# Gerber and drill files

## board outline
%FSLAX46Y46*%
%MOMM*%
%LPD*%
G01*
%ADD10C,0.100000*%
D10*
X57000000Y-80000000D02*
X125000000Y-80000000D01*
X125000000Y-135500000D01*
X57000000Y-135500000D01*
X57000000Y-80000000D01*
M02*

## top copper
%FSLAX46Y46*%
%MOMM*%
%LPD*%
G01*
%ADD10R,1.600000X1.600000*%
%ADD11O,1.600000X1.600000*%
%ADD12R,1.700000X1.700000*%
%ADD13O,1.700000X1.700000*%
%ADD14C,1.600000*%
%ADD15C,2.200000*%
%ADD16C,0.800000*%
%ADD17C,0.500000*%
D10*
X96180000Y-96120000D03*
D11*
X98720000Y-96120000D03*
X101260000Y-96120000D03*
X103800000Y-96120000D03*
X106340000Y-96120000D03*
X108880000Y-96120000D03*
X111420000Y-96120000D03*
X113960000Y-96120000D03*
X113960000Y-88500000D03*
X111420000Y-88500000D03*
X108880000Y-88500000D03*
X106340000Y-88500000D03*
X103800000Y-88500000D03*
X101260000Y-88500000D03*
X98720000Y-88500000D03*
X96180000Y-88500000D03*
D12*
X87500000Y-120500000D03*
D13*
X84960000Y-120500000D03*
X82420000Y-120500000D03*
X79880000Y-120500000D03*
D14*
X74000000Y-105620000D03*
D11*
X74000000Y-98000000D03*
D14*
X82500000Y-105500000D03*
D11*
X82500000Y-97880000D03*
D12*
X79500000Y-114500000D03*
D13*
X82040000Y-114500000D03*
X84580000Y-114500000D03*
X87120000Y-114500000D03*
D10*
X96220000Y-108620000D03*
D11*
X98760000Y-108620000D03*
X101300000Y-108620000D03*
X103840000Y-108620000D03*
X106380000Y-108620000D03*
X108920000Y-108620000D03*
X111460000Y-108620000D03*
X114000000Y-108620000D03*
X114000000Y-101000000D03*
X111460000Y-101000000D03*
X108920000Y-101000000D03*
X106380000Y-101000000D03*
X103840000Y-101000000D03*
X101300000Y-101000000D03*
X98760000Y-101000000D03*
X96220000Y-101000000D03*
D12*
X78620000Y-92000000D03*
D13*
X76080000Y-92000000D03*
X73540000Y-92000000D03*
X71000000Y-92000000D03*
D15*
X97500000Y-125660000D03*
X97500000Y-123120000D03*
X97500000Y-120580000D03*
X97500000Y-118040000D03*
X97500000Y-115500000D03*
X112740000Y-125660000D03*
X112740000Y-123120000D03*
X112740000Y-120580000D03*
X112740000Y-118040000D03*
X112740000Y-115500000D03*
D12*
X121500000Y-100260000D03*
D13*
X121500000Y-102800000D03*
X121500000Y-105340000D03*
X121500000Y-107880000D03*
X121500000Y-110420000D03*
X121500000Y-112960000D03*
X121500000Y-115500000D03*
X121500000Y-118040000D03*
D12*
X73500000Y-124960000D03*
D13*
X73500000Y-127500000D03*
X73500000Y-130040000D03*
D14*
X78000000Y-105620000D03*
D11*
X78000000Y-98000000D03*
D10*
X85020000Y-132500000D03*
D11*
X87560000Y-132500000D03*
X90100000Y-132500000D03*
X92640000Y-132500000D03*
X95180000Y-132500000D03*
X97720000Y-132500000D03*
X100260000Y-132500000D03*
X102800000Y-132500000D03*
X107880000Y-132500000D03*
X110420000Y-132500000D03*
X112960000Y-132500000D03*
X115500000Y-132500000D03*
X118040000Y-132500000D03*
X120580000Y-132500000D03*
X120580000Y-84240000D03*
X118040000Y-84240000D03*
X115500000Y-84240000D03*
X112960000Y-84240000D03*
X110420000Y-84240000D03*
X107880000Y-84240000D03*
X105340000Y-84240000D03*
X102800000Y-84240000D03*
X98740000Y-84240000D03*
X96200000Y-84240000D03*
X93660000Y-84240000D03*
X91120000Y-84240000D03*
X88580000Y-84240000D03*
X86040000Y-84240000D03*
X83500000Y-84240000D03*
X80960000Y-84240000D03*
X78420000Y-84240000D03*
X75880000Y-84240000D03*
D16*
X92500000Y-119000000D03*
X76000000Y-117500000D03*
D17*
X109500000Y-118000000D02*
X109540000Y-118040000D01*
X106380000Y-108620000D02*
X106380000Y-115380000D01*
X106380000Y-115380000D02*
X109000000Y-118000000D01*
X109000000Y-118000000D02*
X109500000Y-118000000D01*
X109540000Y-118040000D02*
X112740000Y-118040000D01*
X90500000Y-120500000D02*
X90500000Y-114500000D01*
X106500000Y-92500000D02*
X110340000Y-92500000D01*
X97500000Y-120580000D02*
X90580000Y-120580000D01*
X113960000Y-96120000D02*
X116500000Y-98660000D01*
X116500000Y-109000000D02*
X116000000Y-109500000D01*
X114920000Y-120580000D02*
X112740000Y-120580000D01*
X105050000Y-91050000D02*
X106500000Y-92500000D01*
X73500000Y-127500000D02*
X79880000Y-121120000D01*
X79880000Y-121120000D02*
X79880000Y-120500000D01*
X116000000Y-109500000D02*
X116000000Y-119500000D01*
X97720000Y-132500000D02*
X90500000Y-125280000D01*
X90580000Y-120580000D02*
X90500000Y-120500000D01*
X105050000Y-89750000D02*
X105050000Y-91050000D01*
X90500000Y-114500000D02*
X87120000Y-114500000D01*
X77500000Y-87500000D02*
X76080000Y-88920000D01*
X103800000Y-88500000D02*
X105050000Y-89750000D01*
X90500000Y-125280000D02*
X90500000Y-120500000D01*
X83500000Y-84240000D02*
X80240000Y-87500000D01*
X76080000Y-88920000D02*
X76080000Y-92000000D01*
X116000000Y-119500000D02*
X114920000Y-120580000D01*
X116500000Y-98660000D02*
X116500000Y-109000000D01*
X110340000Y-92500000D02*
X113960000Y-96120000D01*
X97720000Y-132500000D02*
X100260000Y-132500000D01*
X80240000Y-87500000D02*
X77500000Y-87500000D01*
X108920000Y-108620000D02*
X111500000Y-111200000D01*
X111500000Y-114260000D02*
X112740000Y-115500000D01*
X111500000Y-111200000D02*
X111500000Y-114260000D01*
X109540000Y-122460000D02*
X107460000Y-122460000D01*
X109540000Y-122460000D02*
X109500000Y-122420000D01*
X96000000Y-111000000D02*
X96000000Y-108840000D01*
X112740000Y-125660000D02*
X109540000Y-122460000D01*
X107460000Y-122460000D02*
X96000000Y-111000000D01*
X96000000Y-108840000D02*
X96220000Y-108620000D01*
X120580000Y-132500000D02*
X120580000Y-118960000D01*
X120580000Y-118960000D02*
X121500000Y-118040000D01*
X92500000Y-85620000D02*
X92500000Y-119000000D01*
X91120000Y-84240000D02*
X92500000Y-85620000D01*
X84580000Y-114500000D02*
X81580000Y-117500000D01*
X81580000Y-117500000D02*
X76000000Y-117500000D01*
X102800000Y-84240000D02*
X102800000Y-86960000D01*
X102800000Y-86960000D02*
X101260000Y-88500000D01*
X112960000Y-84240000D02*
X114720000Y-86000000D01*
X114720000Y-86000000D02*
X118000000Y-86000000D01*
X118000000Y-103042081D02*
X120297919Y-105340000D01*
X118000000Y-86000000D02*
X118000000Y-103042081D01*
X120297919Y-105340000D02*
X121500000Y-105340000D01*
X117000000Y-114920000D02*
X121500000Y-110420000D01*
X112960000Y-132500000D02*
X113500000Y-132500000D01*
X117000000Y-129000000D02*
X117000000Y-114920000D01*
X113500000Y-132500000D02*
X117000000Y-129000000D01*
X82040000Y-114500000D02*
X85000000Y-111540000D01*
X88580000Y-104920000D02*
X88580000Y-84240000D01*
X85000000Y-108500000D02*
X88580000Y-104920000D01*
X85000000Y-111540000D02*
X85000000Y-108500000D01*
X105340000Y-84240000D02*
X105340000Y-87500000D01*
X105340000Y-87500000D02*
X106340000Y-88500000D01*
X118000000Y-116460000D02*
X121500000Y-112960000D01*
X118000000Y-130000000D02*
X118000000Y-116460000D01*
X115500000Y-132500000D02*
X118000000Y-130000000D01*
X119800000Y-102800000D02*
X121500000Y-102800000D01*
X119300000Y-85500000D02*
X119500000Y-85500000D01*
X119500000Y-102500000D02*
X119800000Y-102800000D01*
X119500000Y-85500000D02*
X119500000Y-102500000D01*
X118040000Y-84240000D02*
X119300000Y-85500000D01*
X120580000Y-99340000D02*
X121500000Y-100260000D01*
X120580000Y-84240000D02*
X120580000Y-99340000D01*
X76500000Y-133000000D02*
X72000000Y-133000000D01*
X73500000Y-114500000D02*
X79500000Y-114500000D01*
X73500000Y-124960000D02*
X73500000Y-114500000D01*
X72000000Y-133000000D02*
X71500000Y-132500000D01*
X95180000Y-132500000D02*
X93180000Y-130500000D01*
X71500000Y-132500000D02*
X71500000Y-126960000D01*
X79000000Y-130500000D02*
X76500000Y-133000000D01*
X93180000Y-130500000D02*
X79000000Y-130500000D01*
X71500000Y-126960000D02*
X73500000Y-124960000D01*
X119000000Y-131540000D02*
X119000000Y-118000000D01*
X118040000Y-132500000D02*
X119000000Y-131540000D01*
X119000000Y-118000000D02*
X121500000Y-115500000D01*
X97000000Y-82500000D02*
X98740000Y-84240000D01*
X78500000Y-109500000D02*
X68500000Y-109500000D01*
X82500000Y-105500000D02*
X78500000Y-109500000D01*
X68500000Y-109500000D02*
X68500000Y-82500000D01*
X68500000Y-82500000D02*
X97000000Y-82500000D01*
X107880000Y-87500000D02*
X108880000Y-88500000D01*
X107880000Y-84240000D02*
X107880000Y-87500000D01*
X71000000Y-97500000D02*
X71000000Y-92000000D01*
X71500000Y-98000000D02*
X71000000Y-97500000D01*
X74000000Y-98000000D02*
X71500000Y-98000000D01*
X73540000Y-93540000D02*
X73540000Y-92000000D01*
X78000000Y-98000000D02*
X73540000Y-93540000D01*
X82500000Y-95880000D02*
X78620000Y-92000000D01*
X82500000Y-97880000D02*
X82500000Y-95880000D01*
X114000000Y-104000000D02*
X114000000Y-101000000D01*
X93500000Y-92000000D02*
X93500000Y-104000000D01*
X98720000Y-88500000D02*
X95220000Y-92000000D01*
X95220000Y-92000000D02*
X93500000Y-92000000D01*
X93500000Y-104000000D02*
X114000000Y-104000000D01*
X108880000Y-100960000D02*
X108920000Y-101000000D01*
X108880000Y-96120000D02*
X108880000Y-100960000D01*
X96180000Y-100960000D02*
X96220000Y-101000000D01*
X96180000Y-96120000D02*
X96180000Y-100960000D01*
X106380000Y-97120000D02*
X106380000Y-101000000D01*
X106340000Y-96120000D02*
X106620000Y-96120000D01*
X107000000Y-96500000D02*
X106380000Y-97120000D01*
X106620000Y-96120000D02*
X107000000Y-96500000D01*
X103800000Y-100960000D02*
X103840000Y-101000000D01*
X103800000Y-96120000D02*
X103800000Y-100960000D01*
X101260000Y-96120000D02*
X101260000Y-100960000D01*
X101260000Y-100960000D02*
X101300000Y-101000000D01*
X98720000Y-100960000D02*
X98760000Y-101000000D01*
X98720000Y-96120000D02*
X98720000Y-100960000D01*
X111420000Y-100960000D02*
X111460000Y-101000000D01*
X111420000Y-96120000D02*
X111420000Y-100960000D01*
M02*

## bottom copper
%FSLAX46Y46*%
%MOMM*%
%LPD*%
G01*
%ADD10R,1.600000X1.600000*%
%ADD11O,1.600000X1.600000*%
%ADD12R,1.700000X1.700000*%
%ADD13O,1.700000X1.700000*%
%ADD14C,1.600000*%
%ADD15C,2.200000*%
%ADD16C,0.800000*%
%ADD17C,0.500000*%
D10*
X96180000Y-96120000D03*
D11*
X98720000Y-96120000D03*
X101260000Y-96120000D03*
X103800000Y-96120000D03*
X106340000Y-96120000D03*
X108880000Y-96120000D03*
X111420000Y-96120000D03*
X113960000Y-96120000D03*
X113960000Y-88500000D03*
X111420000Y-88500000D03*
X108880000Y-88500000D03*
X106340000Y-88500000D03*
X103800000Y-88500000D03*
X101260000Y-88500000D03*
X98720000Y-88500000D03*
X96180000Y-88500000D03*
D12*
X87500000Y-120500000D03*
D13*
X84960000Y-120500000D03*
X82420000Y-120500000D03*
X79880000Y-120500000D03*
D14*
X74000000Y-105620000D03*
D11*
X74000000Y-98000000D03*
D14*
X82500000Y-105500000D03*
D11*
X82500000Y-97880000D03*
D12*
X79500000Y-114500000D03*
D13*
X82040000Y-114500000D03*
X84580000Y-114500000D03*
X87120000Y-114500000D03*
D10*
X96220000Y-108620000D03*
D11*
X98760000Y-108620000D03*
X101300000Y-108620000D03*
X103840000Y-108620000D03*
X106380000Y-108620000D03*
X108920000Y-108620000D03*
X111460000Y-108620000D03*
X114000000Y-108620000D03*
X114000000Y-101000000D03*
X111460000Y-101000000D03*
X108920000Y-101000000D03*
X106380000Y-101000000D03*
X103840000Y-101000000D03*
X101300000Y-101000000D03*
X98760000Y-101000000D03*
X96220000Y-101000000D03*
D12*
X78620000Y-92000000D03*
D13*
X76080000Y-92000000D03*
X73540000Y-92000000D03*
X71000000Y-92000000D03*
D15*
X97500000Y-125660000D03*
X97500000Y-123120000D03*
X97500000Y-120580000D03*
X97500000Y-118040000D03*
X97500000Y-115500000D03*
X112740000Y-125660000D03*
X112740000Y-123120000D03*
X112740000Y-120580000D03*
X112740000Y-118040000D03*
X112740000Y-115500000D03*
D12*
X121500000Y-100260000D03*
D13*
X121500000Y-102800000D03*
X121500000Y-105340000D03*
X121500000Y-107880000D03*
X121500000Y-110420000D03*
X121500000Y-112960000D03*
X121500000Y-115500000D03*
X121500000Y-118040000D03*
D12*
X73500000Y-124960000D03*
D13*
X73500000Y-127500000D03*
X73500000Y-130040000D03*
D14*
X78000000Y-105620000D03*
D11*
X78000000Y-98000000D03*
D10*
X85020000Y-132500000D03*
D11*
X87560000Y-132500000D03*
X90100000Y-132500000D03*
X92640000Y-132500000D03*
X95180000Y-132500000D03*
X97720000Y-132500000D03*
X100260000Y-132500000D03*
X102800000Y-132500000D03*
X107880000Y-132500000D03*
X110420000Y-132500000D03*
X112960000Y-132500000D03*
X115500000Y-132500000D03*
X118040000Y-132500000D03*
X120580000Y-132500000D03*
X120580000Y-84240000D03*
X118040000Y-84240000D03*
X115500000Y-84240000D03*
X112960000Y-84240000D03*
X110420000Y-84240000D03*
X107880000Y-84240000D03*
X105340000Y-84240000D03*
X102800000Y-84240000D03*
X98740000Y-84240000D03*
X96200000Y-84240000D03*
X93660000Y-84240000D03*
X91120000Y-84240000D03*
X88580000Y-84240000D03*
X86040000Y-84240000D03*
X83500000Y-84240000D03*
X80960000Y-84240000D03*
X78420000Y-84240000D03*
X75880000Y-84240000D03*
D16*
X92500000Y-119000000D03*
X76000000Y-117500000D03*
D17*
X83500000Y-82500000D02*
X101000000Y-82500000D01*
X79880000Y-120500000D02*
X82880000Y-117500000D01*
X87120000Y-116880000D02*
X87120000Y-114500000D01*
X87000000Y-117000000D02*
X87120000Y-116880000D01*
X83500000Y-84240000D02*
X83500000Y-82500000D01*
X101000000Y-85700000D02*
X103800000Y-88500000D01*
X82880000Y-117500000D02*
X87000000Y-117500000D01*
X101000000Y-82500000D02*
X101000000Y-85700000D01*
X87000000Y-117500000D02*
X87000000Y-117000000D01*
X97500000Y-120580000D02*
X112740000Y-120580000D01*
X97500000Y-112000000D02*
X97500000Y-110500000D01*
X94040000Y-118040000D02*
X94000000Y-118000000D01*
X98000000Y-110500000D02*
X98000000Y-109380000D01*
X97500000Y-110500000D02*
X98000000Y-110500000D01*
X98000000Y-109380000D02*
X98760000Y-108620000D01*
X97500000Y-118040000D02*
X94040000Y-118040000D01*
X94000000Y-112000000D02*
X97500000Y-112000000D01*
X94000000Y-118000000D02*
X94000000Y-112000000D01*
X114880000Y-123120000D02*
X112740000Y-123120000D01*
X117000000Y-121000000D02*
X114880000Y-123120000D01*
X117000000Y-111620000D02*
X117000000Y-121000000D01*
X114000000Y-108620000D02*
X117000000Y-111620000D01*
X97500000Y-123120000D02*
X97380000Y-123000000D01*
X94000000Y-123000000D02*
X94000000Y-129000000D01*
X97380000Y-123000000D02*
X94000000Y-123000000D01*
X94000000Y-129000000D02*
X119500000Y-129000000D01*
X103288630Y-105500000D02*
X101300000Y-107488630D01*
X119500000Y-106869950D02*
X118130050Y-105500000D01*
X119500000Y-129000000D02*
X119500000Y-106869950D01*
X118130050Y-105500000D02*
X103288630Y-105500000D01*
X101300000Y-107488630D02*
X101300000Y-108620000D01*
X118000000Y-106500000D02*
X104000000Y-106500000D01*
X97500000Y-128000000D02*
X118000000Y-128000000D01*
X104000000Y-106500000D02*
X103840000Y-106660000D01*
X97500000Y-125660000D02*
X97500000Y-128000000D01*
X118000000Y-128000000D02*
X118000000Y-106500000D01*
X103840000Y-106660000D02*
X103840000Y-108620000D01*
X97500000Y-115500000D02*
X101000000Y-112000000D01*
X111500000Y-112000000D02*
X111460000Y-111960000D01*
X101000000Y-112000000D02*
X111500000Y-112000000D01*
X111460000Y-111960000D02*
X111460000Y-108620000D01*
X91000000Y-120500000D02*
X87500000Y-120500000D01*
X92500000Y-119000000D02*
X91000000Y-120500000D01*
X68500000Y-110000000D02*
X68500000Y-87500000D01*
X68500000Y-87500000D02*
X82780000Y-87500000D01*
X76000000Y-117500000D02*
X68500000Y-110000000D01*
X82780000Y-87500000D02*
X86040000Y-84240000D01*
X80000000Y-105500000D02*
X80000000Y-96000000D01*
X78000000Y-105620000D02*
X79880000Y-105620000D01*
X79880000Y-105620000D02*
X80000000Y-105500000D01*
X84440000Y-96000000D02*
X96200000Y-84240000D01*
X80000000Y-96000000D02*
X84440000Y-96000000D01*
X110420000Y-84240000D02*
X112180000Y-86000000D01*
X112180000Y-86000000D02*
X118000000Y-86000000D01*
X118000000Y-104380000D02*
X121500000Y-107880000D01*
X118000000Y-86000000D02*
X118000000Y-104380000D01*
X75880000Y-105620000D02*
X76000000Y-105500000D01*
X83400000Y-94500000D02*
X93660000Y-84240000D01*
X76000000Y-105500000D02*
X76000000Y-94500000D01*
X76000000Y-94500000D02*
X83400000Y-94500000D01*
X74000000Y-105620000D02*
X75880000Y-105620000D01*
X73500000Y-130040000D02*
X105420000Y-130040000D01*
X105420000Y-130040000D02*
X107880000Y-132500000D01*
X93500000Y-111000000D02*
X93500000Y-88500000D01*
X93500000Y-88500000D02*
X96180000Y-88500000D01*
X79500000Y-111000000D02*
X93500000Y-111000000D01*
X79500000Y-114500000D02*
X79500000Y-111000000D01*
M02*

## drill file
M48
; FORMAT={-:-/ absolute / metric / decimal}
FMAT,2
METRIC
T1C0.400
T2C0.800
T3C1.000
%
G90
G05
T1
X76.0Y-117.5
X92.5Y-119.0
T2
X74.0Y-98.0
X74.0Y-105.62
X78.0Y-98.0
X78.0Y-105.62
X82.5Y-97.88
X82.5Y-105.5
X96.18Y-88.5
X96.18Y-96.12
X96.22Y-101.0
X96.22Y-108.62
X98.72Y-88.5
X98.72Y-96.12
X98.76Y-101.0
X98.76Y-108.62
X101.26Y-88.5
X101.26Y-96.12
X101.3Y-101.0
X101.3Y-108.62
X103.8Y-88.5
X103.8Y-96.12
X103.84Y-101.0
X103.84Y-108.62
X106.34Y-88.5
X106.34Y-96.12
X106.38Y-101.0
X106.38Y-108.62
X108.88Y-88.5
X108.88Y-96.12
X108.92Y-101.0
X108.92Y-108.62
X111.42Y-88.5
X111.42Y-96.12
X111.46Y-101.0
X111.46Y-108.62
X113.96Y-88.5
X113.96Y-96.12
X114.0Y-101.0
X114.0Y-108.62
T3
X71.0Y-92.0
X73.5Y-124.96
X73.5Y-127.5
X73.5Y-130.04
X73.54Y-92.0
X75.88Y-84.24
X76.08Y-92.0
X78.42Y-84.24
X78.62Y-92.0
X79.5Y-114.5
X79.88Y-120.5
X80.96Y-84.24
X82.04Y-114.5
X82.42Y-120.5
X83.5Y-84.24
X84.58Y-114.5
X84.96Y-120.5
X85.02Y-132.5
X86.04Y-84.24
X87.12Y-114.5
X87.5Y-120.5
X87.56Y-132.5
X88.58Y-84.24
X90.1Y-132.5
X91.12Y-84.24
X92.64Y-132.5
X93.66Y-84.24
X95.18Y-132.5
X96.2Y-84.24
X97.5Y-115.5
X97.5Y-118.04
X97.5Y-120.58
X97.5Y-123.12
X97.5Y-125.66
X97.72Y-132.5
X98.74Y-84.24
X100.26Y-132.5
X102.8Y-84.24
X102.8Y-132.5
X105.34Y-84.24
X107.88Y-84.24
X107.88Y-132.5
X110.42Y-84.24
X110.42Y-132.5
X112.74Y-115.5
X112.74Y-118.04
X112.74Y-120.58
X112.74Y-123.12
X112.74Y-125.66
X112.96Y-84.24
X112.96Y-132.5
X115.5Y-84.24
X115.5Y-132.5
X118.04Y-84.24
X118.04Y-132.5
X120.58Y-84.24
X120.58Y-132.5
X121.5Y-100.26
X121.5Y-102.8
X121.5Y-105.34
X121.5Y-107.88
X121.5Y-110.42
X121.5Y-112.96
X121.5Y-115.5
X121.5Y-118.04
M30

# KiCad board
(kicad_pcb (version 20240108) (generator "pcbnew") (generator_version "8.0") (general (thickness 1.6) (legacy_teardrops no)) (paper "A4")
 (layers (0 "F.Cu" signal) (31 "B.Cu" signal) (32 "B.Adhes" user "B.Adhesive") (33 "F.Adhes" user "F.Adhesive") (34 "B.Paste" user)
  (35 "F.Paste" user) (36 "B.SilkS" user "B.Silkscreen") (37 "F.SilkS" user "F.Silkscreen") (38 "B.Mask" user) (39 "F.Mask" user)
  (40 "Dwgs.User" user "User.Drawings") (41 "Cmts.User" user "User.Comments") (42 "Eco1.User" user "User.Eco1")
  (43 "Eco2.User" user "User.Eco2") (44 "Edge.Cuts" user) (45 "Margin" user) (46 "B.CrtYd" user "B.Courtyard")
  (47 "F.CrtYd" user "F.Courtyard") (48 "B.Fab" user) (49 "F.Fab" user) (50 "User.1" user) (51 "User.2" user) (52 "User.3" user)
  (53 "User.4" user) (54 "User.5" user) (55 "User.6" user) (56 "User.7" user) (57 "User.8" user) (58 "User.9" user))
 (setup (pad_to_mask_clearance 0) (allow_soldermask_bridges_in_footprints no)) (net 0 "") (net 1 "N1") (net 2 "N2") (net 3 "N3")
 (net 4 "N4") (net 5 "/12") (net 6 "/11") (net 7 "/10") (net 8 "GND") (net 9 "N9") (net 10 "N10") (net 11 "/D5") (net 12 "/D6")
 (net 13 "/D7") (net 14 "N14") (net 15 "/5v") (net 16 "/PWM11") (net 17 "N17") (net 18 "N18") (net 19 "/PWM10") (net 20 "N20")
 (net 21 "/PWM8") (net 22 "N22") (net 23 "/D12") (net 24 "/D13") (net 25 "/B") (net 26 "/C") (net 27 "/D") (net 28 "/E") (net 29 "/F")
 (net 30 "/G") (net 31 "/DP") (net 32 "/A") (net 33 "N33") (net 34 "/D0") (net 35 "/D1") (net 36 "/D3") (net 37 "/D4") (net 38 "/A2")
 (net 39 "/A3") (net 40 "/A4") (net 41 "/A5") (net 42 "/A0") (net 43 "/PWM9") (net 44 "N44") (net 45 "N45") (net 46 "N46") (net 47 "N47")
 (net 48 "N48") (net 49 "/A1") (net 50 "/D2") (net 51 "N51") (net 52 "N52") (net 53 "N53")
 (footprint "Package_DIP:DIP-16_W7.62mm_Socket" (layer "F.Cu") (at 96.18 96.12 90)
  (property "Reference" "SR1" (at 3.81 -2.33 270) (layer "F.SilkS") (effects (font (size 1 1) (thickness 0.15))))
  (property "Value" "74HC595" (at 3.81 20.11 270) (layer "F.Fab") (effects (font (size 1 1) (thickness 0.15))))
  (pad "1" thru_hole rect (at 0 0 90) (size 1.6 1.6) (drill 0.8) (layers "*.Cu" "*.Mask") (remove_unused_layers no) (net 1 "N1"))
  (pad "2" thru_hole oval (at 0 2.54 90) (size 1.6 1.6) (drill 0.8) (layers "*.Cu" "*.Mask") (remove_unused_layers no) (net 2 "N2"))
  (pad "3" thru_hole oval (at 0 5.08 90) (size 1.6 1.6) (drill 0.8) (layers "*.Cu" "*.Mask") (remove_unused_layers no) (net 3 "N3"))
  (pad "4" thru_hole oval (at 0 7.62 90) (size 1.6 1.6) (drill 0.8) (layers "*.Cu" "*.Mask") (remove_unused_layers no) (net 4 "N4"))
  (pad "5" thru_hole oval (at 0 10.16 90) (size 1.6 1.6) (drill 0.8) (layers "*.Cu" "*.Mask") (remove_unused_layers no) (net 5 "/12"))
  (pad "6" thru_hole oval (at 0 12.7 90) (size 1.6 1.6) (drill 0.8) (layers "*.Cu" "*.Mask") (remove_unused_layers no) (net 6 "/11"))
  (pad "7" thru_hole oval (at 0 15.24 90) (size 1.6 1.6) (drill 0.8) (layers "*.Cu" "*.Mask") (remove_unused_layers no) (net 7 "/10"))
  (pad "8" thru_hole oval (at 0 17.78 90) (size 1.6 1.6) (drill 0.8) (layers "*.Cu" "*.Mask") (remove_unused_layers no) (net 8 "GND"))
  (pad "9" thru_hole oval (at 7.62 17.78 90) (size 1.6 1.6) (drill 0.8) (layers "*.Cu" "*.Mask") (remove_unused_layers no) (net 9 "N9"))
  (pad "10" thru_hole oval (at 7.62 15.24 90) (size 1.6 1.6) (drill 0.8) (layers "*.Cu" "*.Mask") (remove_unused_layers no) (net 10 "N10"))
  (pad "11" thru_hole oval (at 7.62 12.7 90) (size 1.6 1.6) (drill 0.8) (layers "*.Cu" "*.Mask") (remove_unused_layers no) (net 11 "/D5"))
  (pad "12" thru_hole oval (at 7.62 10.16 90) (size 1.6 1.6) (drill 0.8) (layers "*.Cu" "*.Mask") (remove_unused_layers no) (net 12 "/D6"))
  (pad "13" thru_hole oval (at 7.62 7.62 90) (size 1.6 1.6) (drill 0.8) (layers "*.Cu" "*.Mask") (remove_unused_layers no) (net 8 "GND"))
  (pad "14" thru_hole oval (at 7.62 5.08 90) (size 1.6 1.6) (drill 0.8) (layers "*.Cu" "*.Mask") (remove_unused_layers no) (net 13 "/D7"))
  (pad "15" thru_hole oval (at 7.62 2.54 90) (size 1.6 1.6) (drill 0.8) (layers "*.Cu" "*.Mask") (remove_unused_layers no) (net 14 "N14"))
  (pad "16" thru_hole oval (at 7.62 0 90) (size 1.6 1.6) (drill 0.8) (layers "*.Cu" "*.Mask") (remove_unused_layers no) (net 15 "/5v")))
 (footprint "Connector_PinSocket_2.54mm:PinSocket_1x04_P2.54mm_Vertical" (layer "F.Cu") (at 87.5 120.5 -90)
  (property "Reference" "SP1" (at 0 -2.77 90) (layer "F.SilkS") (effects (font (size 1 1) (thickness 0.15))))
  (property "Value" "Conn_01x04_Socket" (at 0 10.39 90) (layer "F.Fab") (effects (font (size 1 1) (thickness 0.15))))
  (pad "1" thru_hole rect (at 0 0 270) (size 1.7 1.7) (drill 1) (layers "*.Cu" "*.Mask") (remove_unused_layers no) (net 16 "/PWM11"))
  (pad "2" thru_hole oval (at 0 2.54 270) (size 1.7 1.7) (drill 1) (layers "*.Cu" "*.Mask") (remove_unused_layers no) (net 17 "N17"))
  (pad "3" thru_hole oval (at 0 5.08 270) (size 1.7 1.7) (drill 1) (layers "*.Cu" "*.Mask") (remove_unused_layers no) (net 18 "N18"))
  (pad "4" thru_hole oval (at 0 7.62 270) (size 1.7 1.7) (drill 1) (layers "*.Cu" "*.Mask") (remove_unused_layers no) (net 8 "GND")))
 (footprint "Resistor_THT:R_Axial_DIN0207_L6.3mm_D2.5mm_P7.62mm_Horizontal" (layer "F.Cu") (at 74 105.62 90)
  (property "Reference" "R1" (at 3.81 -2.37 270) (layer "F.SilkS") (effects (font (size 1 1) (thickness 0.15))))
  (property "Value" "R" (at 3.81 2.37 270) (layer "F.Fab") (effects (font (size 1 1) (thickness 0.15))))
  (pad "1" thru_hole circle (at 0 0 90) (size 1.6 1.6) (drill 0.8) (layers "*.Cu" "*.Mask") (remove_unused_layers no) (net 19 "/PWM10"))
  (pad "2" thru_hole oval (at 7.62 0 90) (size 1.6 1.6) (drill 0.8) (layers "*.Cu" "*.Mask") (remove_unused_layers no) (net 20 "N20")))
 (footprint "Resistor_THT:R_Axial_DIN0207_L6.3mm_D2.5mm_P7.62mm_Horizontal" (layer "F.Cu") (at 82.5 105.5 90)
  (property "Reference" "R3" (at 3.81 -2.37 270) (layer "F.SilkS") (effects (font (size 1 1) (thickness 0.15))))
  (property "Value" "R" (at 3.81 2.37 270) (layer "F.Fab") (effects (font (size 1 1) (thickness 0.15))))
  (pad "1" thru_hole circle (at 0 0 90) (size 1.6 1.6) (drill 0.8) (layers "*.Cu" "*.Mask") (remove_unused_layers no) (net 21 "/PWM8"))
  (pad "2" thru_hole oval (at 7.62 0 90) (size 1.6 1.6) (drill 0.8) (layers "*.Cu" "*.Mask") (remove_unused_layers no) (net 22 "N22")))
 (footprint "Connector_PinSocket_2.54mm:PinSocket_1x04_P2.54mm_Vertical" (layer "F.Cu") (at 79.5 114.5 90)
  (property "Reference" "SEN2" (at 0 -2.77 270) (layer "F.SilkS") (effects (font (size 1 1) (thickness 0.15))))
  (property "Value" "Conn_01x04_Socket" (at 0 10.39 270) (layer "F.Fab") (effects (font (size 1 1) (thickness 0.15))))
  (pad "1" thru_hole rect (at 0 0 90) (size 1.7 1.7) (drill 1) (layers "*.Cu" "*.Mask") (remove_unused_layers no) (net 15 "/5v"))
  (pad "2" thru_hole oval (at 0 2.54 90) (size 1.7 1.7) (drill 1) (layers "*.Cu" "*.Mask") (remove_unused_layers no) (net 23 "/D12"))
  (pad "3" thru_hole oval (at 0 5.08 90) (size 1.7 1.7) (drill 1) (layers "*.Cu" "*.Mask") (remove_unused_layers no) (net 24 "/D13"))
  (pad "4" thru_hole oval (at 0 7.62 90) (size 1.7 1.7) (drill 1) (layers "*.Cu" "*.Mask") (remove_unused_layers no) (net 8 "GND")))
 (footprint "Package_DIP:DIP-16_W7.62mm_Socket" (layer "F.Cu") (at 96.22 108.62 90)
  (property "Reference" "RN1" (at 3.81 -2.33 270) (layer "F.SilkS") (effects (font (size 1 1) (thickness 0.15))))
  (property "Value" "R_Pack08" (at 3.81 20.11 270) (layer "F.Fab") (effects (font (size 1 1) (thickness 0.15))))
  (pad "1" thru_hole rect (at 0 0 90) (size 1.6 1.6) (drill 0.8) (layers "*.Cu" "*.Mask") (remove_unused_layers no) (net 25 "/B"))
  (pad "2" thru_hole oval (at 0 2.54 90) (size 1.6 1.6) (drill 0.8) (layers "*.Cu" "*.Mask") (remove_unused_layers no) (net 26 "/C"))
  (pad "3" thru_hole oval (at 0 5.08 90) (size 1.6 1.6) (drill 0.8) (layers "*.Cu" "*.Mask") (remove_unused_layers no) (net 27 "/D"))
  (pad "4" thru_hole oval (at 0 7.62 90) (size 1.6 1.6) (drill 0.8) (layers "*.Cu" "*.Mask") (remove_unused_layers no) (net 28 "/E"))
  (pad "5" thru_hole oval (at 0 10.16 90) (size 1.6 1.6) (drill 0.8) (layers "*.Cu" "*.Mask") (remove_unused_layers no) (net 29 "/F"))
  (pad "6" thru_hole oval (at 0 12.7 90) (size 1.6 1.6) (drill 0.8) (layers "*.Cu" "*.Mask") (remove_unused_layers no) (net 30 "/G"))
  (pad "7" thru_hole oval (at 0 15.24 90) (size 1.6 1.6) (drill 0.8) (layers "*.Cu" "*.Mask") (remove_unused_layers no) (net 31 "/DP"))
  (pad "8" thru_hole oval (at 0 17.78 90) (size 1.6 1.6) (drill 0.8) (layers "*.Cu" "*.Mask") (remove_unused_layers no) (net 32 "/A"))
  (pad "9" thru_hole oval (at 7.62 17.78 90) (size 1.6 1.6) (drill 0.8) (layers "*.Cu" "*.Mask") (remove_unused_layers no) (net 14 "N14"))
  (pad "10" thru_hole oval (at 7.62 15.24 90) (size 1.6 1.6) (drill 0.8) (layers "*.Cu" "*.Mask") (remove_unused_layers no) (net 7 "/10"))
  (pad "11" thru_hole oval (at 7.62 12.7 90) (size 1.6 1.6) (drill 0.8) (layers "*.Cu" "*.Mask") (remove_unused_layers no) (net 6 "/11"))
  (pad "12" thru_hole oval (at 7.62 10.16 90) (size 1.6 1.6) (drill 0.8) (layers "*.Cu" "*.Mask") (remove_unused_layers no) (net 5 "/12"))
  (pad "13" thru_hole oval (at 7.62 7.62 90) (size 1.6 1.6) (drill 0.8) (layers "*.Cu" "*.Mask") (remove_unused_layers no) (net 4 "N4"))
  (pad "14" thru_hole oval (at 7.62 5.08 90) (size 1.6 1.6) (drill 0.8) (layers "*.Cu" "*.Mask") (remove_unused_layers no) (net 3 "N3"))
  (pad "15" thru_hole oval (at 7.62 2.54 90) (size 1.6 1.6) (drill 0.8) (layers "*.Cu" "*.Mask") (remove_unused_layers no) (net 2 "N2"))
  (pad "16" thru_hole oval (at 7.62 0 90) (size 1.6 1.6) (drill 0.8) (layers "*.Cu" "*.Mask") (remove_unused_layers no) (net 1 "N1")))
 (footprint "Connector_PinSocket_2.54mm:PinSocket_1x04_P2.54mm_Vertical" (layer "F.Cu") (at 78.62 92 -90)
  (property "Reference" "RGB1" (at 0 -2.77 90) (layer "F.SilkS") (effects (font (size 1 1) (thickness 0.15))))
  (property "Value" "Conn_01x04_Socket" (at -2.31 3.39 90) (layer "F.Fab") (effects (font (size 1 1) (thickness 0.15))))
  (pad "1" thru_hole rect (at 0 0 270) (size 1.7 1.7) (drill 1) (layers "*.Cu" "*.Mask") (remove_unused_layers no) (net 22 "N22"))
  (pad "2" thru_hole oval (at 0 2.54 270) (size 1.7 1.7) (drill 1) (layers "*.Cu" "*.Mask") (remove_unused_layers no) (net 8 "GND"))
  (pad "3" thru_hole oval (at 0 5.08 270) (size 1.7 1.7) (drill 1) (layers "*.Cu" "*.Mask") (remove_unused_layers no) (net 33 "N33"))
  (pad "4" thru_hole oval (at 0 7.62 270) (size 1.7 1.7) (drill 1) (layers "*.Cu" "*.Mask") (remove_unused_layers no) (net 20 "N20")))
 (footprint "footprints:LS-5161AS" (layer "F.Cu") (at 97.5 125.66 90)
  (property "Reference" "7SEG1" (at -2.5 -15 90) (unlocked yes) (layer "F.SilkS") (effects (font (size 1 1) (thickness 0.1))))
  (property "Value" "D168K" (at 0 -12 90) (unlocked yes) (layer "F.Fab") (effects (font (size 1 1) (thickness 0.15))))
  (pad "1" thru_hole circle (at 0 0 90) (size 2.2 2.2) (drill 1) (layers "*.Cu" "*.Mask") (remove_unused_layers no) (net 28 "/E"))
  (pad "2" thru_hole circle (at 2.54 0 90) (size 2.2 2.2) (drill 1) (layers "*.Cu" "*.Mask") (remove_unused_layers no) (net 27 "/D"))
  (pad "3" thru_hole circle (at 5.08 0 90) (size 2.2 2.2) (drill 1) (layers "*.Cu" "*.Mask") (remove_unused_layers no) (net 8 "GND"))
  (pad "4" thru_hole circle (at 7.62 0 90) (size 2.2 2.2) (drill 1) (layers "*.Cu" "*.Mask") (remove_unused_layers no) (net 26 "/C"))
  (pad "5" thru_hole circle (at 10.16 0 90) (size 2.2 2.2) (drill 1) (layers "*.Cu" "*.Mask") (remove_unused_layers no) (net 31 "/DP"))
  (pad "6" thru_hole circle (at 0 15.24 90) (size 2.2 2.2) (drill 1) (layers "*.Cu" "*.Mask") (remove_unused_layers no) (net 25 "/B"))
  (pad "7" thru_hole circle (at 2.54 15.24 90) (size 2.2 2.2) (drill 1) (layers "*.Cu" "*.Mask") (remove_unused_layers no) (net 32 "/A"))
  (pad "8" thru_hole circle (at 5.08 15.24 90) (size 2.2 2.2) (drill 1) (layers "*.Cu" "*.Mask") (remove_unused_layers no) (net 8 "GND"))
  (pad "9" thru_hole circle (at 7.62 15.24 90) (size 2.2 2.2) (drill 1) (layers "*.Cu" "*.Mask") (remove_unused_layers no) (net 29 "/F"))
  (pad "10" thru_hole circle (at 10.16 15.24 90) (size 2.2 2.2) (drill 1) (layers "*.Cu" "*.Mask") (remove_unused_layers no) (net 30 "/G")))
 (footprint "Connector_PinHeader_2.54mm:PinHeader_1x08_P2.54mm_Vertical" (layer "F.Cu") (at 121.5 100.26)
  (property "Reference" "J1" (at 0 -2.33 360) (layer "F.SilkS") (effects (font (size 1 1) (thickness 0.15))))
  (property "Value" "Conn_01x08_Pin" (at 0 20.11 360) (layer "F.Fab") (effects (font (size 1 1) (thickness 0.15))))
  (pad "1" thru_hole rect (at 0 0) (size 1.7 1.7) (drill 1) (layers "*.Cu" "*.Mask") (remove_unused_layers no) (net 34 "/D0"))
  (pad "2" thru_hole oval (at 0 2.54) (size 1.7 1.7) (drill 1) (layers "*.Cu" "*.Mask") (remove_unused_layers no) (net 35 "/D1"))
  (pad "3" thru_hole oval (at 0 5.08) (size 1.7 1.7) (drill 1) (layers "*.Cu" "*.Mask") (remove_unused_layers no) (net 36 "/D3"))
  (pad "4" thru_hole oval (at 0 7.62) (size 1.7 1.7) (drill 1) (layers "*.Cu" "*.Mask") (remove_unused_layers no) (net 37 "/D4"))
  (pad "5" thru_hole oval (at 0 10.16) (size 1.7 1.7) (drill 1) (layers "*.Cu" "*.Mask") (remove_unused_layers no) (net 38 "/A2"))
  (pad "6" thru_hole oval (at 0 12.7) (size 1.7 1.7) (drill 1) (layers "*.Cu" "*.Mask") (remove_unused_layers no) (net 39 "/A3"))
  (pad "7" thru_hole oval (at 0 15.24) (size 1.7 1.7) (drill 1) (layers "*.Cu" "*.Mask") (remove_unused_layers no) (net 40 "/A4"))
  (pad "8" thru_hole oval (at 0 17.78) (size 1.7 1.7) (drill 1) (layers "*.Cu" "*.Mask") (remove_unused_layers no) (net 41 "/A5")))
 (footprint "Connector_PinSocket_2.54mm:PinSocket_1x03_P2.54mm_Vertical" (layer "F.Cu") (at 73.5 124.96)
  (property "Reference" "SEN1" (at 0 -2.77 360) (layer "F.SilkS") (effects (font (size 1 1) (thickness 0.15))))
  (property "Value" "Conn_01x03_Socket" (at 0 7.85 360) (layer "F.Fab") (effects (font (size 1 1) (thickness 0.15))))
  (pad "1" thru_hole rect (at 0 0) (size 1.7 1.7) (drill 1) (layers "*.Cu" "*.Mask") (remove_unused_layers no) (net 15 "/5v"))
  (pad "2" thru_hole oval (at 0 2.54) (size 1.7 1.7) (drill 1) (layers "*.Cu" "*.Mask") (remove_unused_layers no) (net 8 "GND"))
  (pad "3" thru_hole oval (at 0 5.08) (size 1.7 1.7) (drill 1) (layers "*.Cu" "*.Mask") (remove_unused_layers no) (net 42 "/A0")))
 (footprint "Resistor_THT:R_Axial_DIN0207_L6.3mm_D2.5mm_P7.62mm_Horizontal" (layer "F.Cu") (at 78 105.62 90)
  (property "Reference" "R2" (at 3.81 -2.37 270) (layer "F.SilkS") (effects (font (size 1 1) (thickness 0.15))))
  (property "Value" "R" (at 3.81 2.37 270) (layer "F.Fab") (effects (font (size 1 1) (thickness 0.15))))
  (pad "1" thru_hole circle (at 0 0 90) (size 1.6 1.6) (drill 0.8) (layers "*.Cu" "*.Mask") (remove_unused_layers no) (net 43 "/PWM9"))
  (pad "2" thru_hole oval (at 7.62 0 90) (size 1.6 1.6) (drill 0.8) (layers "*.Cu" "*.Mask") (remove_unused_layers no) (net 33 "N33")))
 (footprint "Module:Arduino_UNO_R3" (layer "B.Cu") (at 85.02 132.5)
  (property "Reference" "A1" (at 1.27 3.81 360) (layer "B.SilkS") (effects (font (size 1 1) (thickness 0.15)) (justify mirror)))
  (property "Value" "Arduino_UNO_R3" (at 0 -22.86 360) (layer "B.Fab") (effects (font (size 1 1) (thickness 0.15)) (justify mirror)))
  (pad "1" thru_hole rect (at 0 0 270) (size 1.6 1.6) (drill 1) (layers "*.Cu" "*.Mask") (remove_unused_layers no) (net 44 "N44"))
  (pad "2" thru_hole oval (at 2.54 0 270) (size 1.6 1.6) (drill 1) (layers "*.Cu" "*.Mask") (remove_unused_layers no) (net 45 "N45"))
  (pad "3" thru_hole oval (at 5.08 0 270) (size 1.6 1.6) (drill 1) (layers "*.Cu" "*.Mask") (remove_unused_layers no) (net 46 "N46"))
  (pad "4" thru_hole oval (at 7.62 0 270) (size 1.6 1.6) (drill 1) (layers "*.Cu" "*.Mask") (remove_unused_layers no) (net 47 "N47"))
  (pad "5" thru_hole oval (at 10.16 0 270) (size 1.6 1.6) (drill 1) (layers "*.Cu" "*.Mask") (remove_unused_layers no) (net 15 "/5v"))
  (pad "6" thru_hole oval (at 12.7 0 270) (size 1.6 1.6) (drill 1) (layers "*.Cu" "*.Mask") (remove_unused_layers no) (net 8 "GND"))
  (pad "7" thru_hole oval (at 15.24 0 270) (size 1.6 1.6) (drill 1) (layers "*.Cu" "*.Mask") (remove_unused_layers no) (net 8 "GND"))
  (pad "8" thru_hole oval (at 17.78 0 270) (size 1.6 1.6) (drill 1) (layers "*.Cu" "*.Mask") (remove_unused_layers no) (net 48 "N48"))
  (pad "9" thru_hole oval (at 22.86 0 270) (size 1.6 1.6) (drill 1) (layers "*.Cu" "*.Mask") (remove_unused_layers no) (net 42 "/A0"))
  (pad "10" thru_hole oval (at 25.4 0 270) (size 1.6 1.6) (drill 1) (layers "*.Cu" "*.Mask") (remove_unused_layers no) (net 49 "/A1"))
  (pad "11" thru_hole oval (at 27.94 0 270) (size 1.6 1.6) (drill 1) (layers "*.Cu" "*.Mask") (remove_unused_layers no) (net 38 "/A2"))
  (pad "12" thru_hole oval (at 30.48 0 270) (size 1.6 1.6) (drill 1) (layers "*.Cu" "*.Mask") (remove_unused_layers no) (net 39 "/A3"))
  (pad "13" thru_hole oval (at 33.02 0 270) (size 1.6 1.6) (drill 1) (layers "*.Cu" "*.Mask") (remove_unused_layers no) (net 40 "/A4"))
  (pad "14" thru_hole oval (at 35.56 0 270) (size 1.6 1.6) (drill 1) (layers "*.Cu" "*.Mask") (remove_unused_layers no) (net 41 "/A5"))
  (pad "15" thru_hole oval (at 35.56 -48.26 270) (size 1.6 1.6) (drill 1) (layers "*.Cu" "*.Mask") (remove_unused_layers no) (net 34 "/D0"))
  (pad "16" thru_hole oval (at 33.02 -48.26 270) (size 1.6 1.6) (drill 1) (layers "*.Cu" "*.Mask") (remove_unused_layers no) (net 35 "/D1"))
  (pad "17" thru_hole oval (at 30.48 -48.26 270) (size 1.6 1.6) (drill 1) (layers "*.Cu" "*.Mask") (remove_unused_layers no) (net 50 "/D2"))
  (pad "18" thru_hole oval (at 27.94 -48.26 270) (size 1.6 1.6) (drill 1) (layers "*.Cu" "*.Mask") (remove_unused_layers no) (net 36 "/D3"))
  (pad "19" thru_hole oval (at 25.4 -48.26 270) (size 1.6 1.6) (drill 1) (layers "*.Cu" "*.Mask") (remove_unused_layers no) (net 37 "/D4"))
  (pad "20" thru_hole oval (at 22.86 -48.26 270) (size 1.6 1.6) (drill 1) (layers "*.Cu" "*.Mask") (remove_unused_layers no) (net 11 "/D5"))
  (pad "21" thru_hole oval (at 20.32 -48.26 270) (size 1.6 1.6) (drill 1) (layers "*.Cu" "*.Mask") (remove_unused_layers no) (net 12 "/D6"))
  (pad "22" thru_hole oval (at 17.78 -48.26 270) (size 1.6 1.6) (drill 1) (layers "*.Cu" "*.Mask") (remove_unused_layers no) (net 13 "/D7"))
  (pad "23" thru_hole oval (at 13.72 -48.26 270) (size 1.6 1.6) (drill 1) (layers "*.Cu" "*.Mask") (remove_unused_layers no)
   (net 21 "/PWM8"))
  (pad "24" thru_hole oval (at 11.18 -48.26 270) (size 1.6 1.6) (drill 1) (layers "*.Cu" "*.Mask") (remove_unused_layers no)
   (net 43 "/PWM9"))
  (pad "25" thru_hole oval (at 8.64 -48.26 270) (size 1.6 1.6) (drill 1) (layers "*.Cu" "*.Mask") (remove_unused_layers no)
   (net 19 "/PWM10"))
  (pad "26" thru_hole oval (at 6.1 -48.26 270) (size 1.6 1.6) (drill 1) (layers "*.Cu" "*.Mask") (remove_unused_layers no) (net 16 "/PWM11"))
  (pad "27" thru_hole oval (at 3.56 -48.26 270) (size 1.6 1.6) (drill 1) (layers "*.Cu" "*.Mask") (remove_unused_layers no) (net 23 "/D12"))
  (pad "28" thru_hole oval (at 1.02 -48.26 270) (size 1.6 1.6) (drill 1) (layers "*.Cu" "*.Mask") (remove_unused_layers no) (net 24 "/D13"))
  (pad "29" thru_hole oval (at -1.52 -48.26 270) (size 1.6 1.6) (drill 1) (layers "*.Cu" "*.Mask") (remove_unused_layers no) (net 8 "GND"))
  (pad "30" thru_hole oval (at -4.06 -48.26 270) (size 1.6 1.6) (drill 1) (layers "*.Cu" "*.Mask") (remove_unused_layers no) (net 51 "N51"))
  (pad "31" thru_hole oval (at -6.6 -48.26 270) (size 1.6 1.6) (drill 1) (layers "*.Cu" "*.Mask") (remove_unused_layers no) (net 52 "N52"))
  (pad "32" thru_hole oval (at -9.14 -48.26 270) (size 1.6 1.6) (drill 1) (layers "*.Cu" "*.Mask") (remove_unused_layers no) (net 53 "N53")))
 (gr_rect (start 57 80) (end 125 135.5) (stroke (width 0.1) (type default)) (fill none) (layer "Edge.Cuts"))
 (segment (start 109.5 118) (end 109.54 118.04) (width 0.5) (layer "F.Cu") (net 29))
 (segment (start 106.38 108.62) (end 106.38 115.38) (width 0.5) (layer "F.Cu") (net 29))
 (segment (start 106.38 115.38) (end 109 118) (width 0.5) (layer "F.Cu") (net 29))
 (segment (start 109 118) (end 109.5 118) (width 0.5) (layer "F.Cu") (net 29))
 (segment (start 109.54 118.04) (end 112.74 118.04) (width 0.5) (layer "F.Cu") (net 29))
 (segment (start 90.5 120.5) (end 90.5 114.5) (width 0.5) (layer "F.Cu") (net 8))
 (segment (start 106.5 92.5) (end 110.34 92.5) (width 0.5) (layer "F.Cu") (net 8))
 (segment (start 97.5 120.58) (end 90.58 120.58) (width 0.5) (layer "F.Cu") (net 8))
 (segment (start 113.96 96.12) (end 116.5 98.66) (width 0.5) (layer "F.Cu") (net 8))
 (segment (start 116.5 109) (end 116 109.5) (width 0.5) (layer "F.Cu") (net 8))
 (segment (start 114.92 120.58) (end 112.74 120.58) (width 0.5) (layer "F.Cu") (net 8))
 (segment (start 105.05 91.05) (end 106.5 92.5) (width 0.5) (layer "F.Cu") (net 8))
 (segment (start 73.5 127.5) (end 79.88 121.12) (width 0.5) (layer "F.Cu") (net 8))
 (segment (start 79.88 121.12) (end 79.88 120.5) (width 0.5) (layer "F.Cu") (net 8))
 (segment (start 116 109.5) (end 116 119.5) (width 0.5) (layer "F.Cu") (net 8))
 (segment (start 97.72 132.5) (end 90.5 125.28) (width 0.5) (layer "F.Cu") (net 8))
 (segment (start 90.58 120.58) (end 90.5 120.5) (width 0.5) (layer "F.Cu") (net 8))
 (segment (start 105.05 89.75) (end 105.05 91.05) (width 0.5) (layer "F.Cu") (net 8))
 (segment (start 90.5 114.5) (end 87.12 114.5) (width 0.5) (layer "F.Cu") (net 8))
 (segment (start 77.5 87.5) (end 76.08 88.92) (width 0.5) (layer "F.Cu") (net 8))
 (segment (start 103.8 88.5) (end 105.05 89.75) (width 0.5) (layer "F.Cu") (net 8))
 (segment (start 90.5 125.28) (end 90.5 120.5) (width 0.5) (layer "F.Cu") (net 8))
 (segment (start 83.5 84.24) (end 80.24 87.5) (width 0.5) (layer "F.Cu") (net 8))
 (segment (start 76.08 88.92) (end 76.08 92) (width 0.5) (layer "F.Cu") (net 8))
 (segment (start 116 119.5) (end 114.92 120.58) (width 0.5) (layer "F.Cu") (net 8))
 (segment (start 116.5 98.66) (end 116.5 109) (width 0.5) (layer "F.Cu") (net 8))
 (segment (start 110.34 92.5) (end 113.96 96.12) (width 0.5) (layer "F.Cu") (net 8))
 (segment (start 97.72 132.5) (end 100.26 132.5) (width 0.5) (layer "F.Cu") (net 8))
 (segment (start 80.24 87.5) (end 77.5 87.5) (width 0.5) (layer "F.Cu") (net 8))
 (segment (start 83.5 82.5) (end 101 82.5) (width 0.5) (layer "B.Cu") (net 8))
 (segment (start 79.88 120.5) (end 82.88 117.5) (width 0.5) (layer "B.Cu") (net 8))
 (segment (start 87.12 116.88) (end 87.12 114.5) (width 0.5) (layer "B.Cu") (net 8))
 (segment (start 87 117) (end 87.12 116.88) (width 0.5) (layer "B.Cu") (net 8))
 (segment (start 83.5 84.24) (end 83.5 82.5) (width 0.5) (layer "B.Cu") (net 8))
 (segment (start 101 85.7) (end 103.8 88.5) (width 0.5) (layer "B.Cu") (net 8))
 (segment (start 82.88 117.5) (end 87 117.5) (width 0.5) (layer "B.Cu") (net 8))
 (segment (start 101 82.5) (end 101 85.7) (width 0.5) (layer "B.Cu") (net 8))
 (segment (start 87 117.5) (end 87 117) (width 0.5) (layer "B.Cu") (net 8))
 (segment (start 97.5 120.58) (end 112.74 120.58) (width 0.5) (layer "B.Cu") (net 8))
 (segment (start 108.92 108.62) (end 111.5 111.2) (width 0.5) (layer "F.Cu") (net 30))
 (segment (start 111.5 114.26) (end 112.74 115.5) (width 0.5) (layer "F.Cu") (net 30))
 (segment (start 111.5 111.2) (end 111.5 114.26) (width 0.5) (layer "F.Cu") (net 30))
 (segment (start 109.54 122.46) (end 107.46 122.46) (width 0.5) (layer "F.Cu") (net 25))
 (segment (start 109.54 122.46) (end 109.5 122.42) (width 0.5) (layer "F.Cu") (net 25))
 (segment (start 96 111) (end 96 108.84) (width 0.5) (layer "F.Cu") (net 25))
 (segment (start 112.74 125.66) (end 109.54 122.46) (width 0.5) (layer "F.Cu") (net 25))
 (segment (start 107.46 122.46) (end 96 111) (width 0.5) (layer "F.Cu") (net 25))
 (segment (start 96 108.84) (end 96.22 108.62) (width 0.5) (layer "F.Cu") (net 25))
 (segment (start 97.5 112) (end 97.5 110.5) (width 0.5) (layer "B.Cu") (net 26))
 (segment (start 94.04 118.04) (end 94 118) (width 0.5) (layer "B.Cu") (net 26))
 (segment (start 98 110.5) (end 98 109.38) (width 0.5) (layer "B.Cu") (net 26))
 (segment (start 97.5 110.5) (end 98 110.5) (width 0.5) (layer "B.Cu") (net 26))
 (segment (start 98 109.38) (end 98.76 108.62) (width 0.5) (layer "B.Cu") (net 26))
 (segment (start 97.5 118.04) (end 94.04 118.04) (width 0.5) (layer "B.Cu") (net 26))
 (segment (start 94 112) (end 97.5 112) (width 0.5) (layer "B.Cu") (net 26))
 (segment (start 94 118) (end 94 112) (width 0.5) (layer "B.Cu") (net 26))
 (segment (start 114.88 123.12) (end 112.74 123.12) (width 0.5) (layer "B.Cu") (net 32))
 (segment (start 117 121) (end 114.88 123.12) (width 0.5) (layer "B.Cu") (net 32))
 (segment (start 117 111.62) (end 117 121) (width 0.5) (layer "B.Cu") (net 32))
 (segment (start 114 108.62) (end 117 111.62) (width 0.5) (layer "B.Cu") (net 32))
 (segment (start 97.5 123.12) (end 97.38 123) (width 0.5) (layer "B.Cu") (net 27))
 (segment (start 94 123) (end 94 129) (width 0.5) (layer "B.Cu") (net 27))
 (segment (start 97.38 123) (end 94 123) (width 0.5) (layer "B.Cu") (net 27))
 (segment (start 94 129) (end 119.5 129) (width 0.5) (layer "B.Cu") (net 27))
 (segment (start 103.28863 105.5) (end 101.3 107.48863) (width 0.5) (layer "B.Cu") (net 27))
 (segment (start 119.5 106.86995) (end 118.13005 105.5) (width 0.5) (layer "B.Cu") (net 27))
 (segment (start 119.5 129) (end 119.5 106.86995) (width 0.5) (layer "B.Cu") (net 27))
 (segment (start 118.13005 105.5) (end 103.28863 105.5) (width 0.5) (layer "B.Cu") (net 27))
 (segment (start 101.3 107.48863) (end 101.3 108.62) (width 0.5) (layer "B.Cu") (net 27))
 (segment (start 118 106.5) (end 104 106.5) (width 0.5) (layer "B.Cu") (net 28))
 (segment (start 97.5 128) (end 118 128) (width 0.5) (layer "B.Cu") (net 28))
 (segment (start 104 106.5) (end 103.84 106.66) (width 0.5) (layer "B.Cu") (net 28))
 (segment (start 97.5 125.66) (end 97.5 128) (width 0.5) (layer "B.Cu") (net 28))
 (segment (start 118 128) (end 118 106.5) (width 0.5) (layer "B.Cu") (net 28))
 (segment (start 103.84 106.66) (end 103.84 108.62) (width 0.5) (layer "B.Cu") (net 28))
 (segment (start 97.5 115.5) (end 101 112) (width 0.5) (layer "B.Cu") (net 31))
 (segment (start 111.5 112) (end 111.46 111.96) (width 0.5) (layer "B.Cu") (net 31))
 (segment (start 101 112) (end 111.5 112) (width 0.5) (layer "B.Cu") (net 31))
 (segment (start 111.46 111.96) (end 111.46 108.62) (width 0.5) (layer "B.Cu") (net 31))
 (segment (start 120.58 132.5) (end 120.58 118.96) (width 0.5) (layer "F.Cu") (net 41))
 (segment (start 120.58 118.96) (end 121.5 118.04) (width 0.5) (layer "F.Cu") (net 41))
 (segment (start 92.5 85.62) (end 92.5 119) (width 0.5) (layer "F.Cu") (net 16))
 (segment (start 91.12 84.24) (end 92.5 85.62) (width 0.5) (layer "F.Cu") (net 16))
 (via (at 92.5 119) (size 0.8) (drill 0.4) (layers "F.Cu" "B.Cu") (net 16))
 (segment (start 91 120.5) (end 87.5 120.5) (width 0.5) (layer "B.Cu") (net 16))
 (segment (start 92.5 119) (end 91 120.5) (width 0.5) (layer "B.Cu") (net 16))
 (segment (start 84.58 114.5) (end 81.58 117.5) (width 0.5) (layer "F.Cu") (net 24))
 (segment (start 81.58 117.5) (end 76 117.5) (width 0.5) (layer "F.Cu") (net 24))
 (via (at 76 117.5) (size 0.8) (drill 0.4) (layers "F.Cu" "B.Cu") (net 24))
 (segment (start 68.5 110) (end 68.5 87.5) (width 0.5) (layer "B.Cu") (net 24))
 (segment (start 68.5 87.5) (end 82.78 87.5) (width 0.5) (layer "B.Cu") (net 24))
 (segment (start 76 117.5) (end 68.5 110) (width 0.5) (layer "B.Cu") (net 24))
 (segment (start 82.78 87.5) (end 86.04 84.24) (width 0.5) (layer "B.Cu") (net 24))
 (segment (start 102.8 84.24) (end 102.8 86.96) (width 0.5) (layer "F.Cu") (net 13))
 (segment (start 102.8 86.96) (end 101.26 88.5) (width 0.5) (layer "F.Cu") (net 13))
 (segment (start 80 105.5) (end 80 96) (width 0.5) (layer "B.Cu") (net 43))
 (segment (start 78 105.62) (end 79.88 105.62) (width 0.5) (layer "B.Cu") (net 43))
 (segment (start 79.88 105.62) (end 80 105.5) (width 0.5) (layer "B.Cu") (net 43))
 (segment (start 84.44 96) (end 96.2 84.24) (width 0.5) (layer "B.Cu") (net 43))
 (segment (start 80 96) (end 84.44 96) (width 0.5) (layer "B.Cu") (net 43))
 (segment (start 110.42 84.24) (end 112.18 86) (width 0.5) (layer "B.Cu") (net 37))
 (segment (start 112.18 86) (end 118 86) (width 0.5) (layer "B.Cu") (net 37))
 (segment (start 118 104.38) (end 121.5 107.88) (width 0.5) (layer "B.Cu") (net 37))
 (segment (start 118 86) (end 118 104.38) (width 0.5) (layer "B.Cu") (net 37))
 (segment (start 112.96 84.24) (end 114.72 86) (width 0.5) (layer "F.Cu") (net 36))
 (segment (start 114.72 86) (end 118 86) (width 0.5) (layer "F.Cu") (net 36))
 (segment (start 118 103.042081) (end 120.297919 105.34) (width 0.5) (layer "F.Cu") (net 36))
 (segment (start 118 86) (end 118 103.042081) (width 0.5) (layer "F.Cu") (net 36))
 (segment (start 120.297919 105.34) (end 121.5 105.34) (width 0.5) (layer "F.Cu") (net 36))
 (segment (start 75.88 105.62) (end 76 105.5) (width 0.5) (layer "B.Cu") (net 19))
 (segment (start 83.4 94.5) (end 93.66 84.24) (width 0.5) (layer "B.Cu") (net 19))
 (segment (start 76 105.5) (end 76 94.5) (width 0.5) (layer "B.Cu") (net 19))
 (segment (start 76 94.5) (end 83.4 94.5) (width 0.5) (layer "B.Cu") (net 19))
 (segment (start 74 105.62) (end 75.88 105.62) (width 0.5) (layer "B.Cu") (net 19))
 (segment (start 117 114.92) (end 121.5 110.42) (width 0.5) (layer "F.Cu") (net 38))
 (segment (start 112.96 132.5) (end 113.5 132.5) (width 0.5) (layer "F.Cu") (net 38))
 (segment (start 117 129) (end 117 114.92) (width 0.5) (layer "F.Cu") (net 38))
 (segment (start 113.5 132.5) (end 117 129) (width 0.5) (layer "F.Cu") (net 38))
 (segment (start 82.04 114.5) (end 85 111.54) (width 0.5) (layer "F.Cu") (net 23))
 (segment (start 88.58 104.92) (end 88.58 84.24) (width 0.5) (layer "F.Cu") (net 23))
 (segment (start 85 108.5) (end 88.58 104.92) (width 0.5) (layer "F.Cu") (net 23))
 (segment (start 85 111.54) (end 85 108.5) (width 0.5) (layer "F.Cu") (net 23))
 (segment (start 105.34 84.24) (end 105.34 87.5) (width 0.5) (layer "F.Cu") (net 12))
 (segment (start 105.34 87.5) (end 106.34 88.5) (width 0.5) (layer "F.Cu") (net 12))
 (segment (start 118 116.46) (end 121.5 112.96) (width 0.5) (layer "F.Cu") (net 39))
 (segment (start 118 130) (end 118 116.46) (width 0.5) (layer "F.Cu") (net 39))
 (segment (start 115.5 132.5) (end 118 130) (width 0.5) (layer "F.Cu") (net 39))
 (segment (start 119.8 102.8) (end 121.5 102.8) (width 0.5) (layer "F.Cu") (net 35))
 (segment (start 119.3 85.5) (end 119.5 85.5) (width 0.5) (layer "F.Cu") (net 35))
 (segment (start 119.5 102.5) (end 119.8 102.8) (width 0.5) (layer "F.Cu") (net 35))
 (segment (start 119.5 85.5) (end 119.5 102.5) (width 0.5) (layer "F.Cu") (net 35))
 (segment (start 118.04 84.24) (end 119.3 85.5) (width 0.5) (layer "F.Cu") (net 35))
 (segment (start 73.5 130.04) (end 105.42 130.04) (width 0.5) (layer "B.Cu") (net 42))
 (segment (start 105.42 130.04) (end 107.88 132.5) (width 0.5) (layer "B.Cu") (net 42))
 (segment (start 120.58 99.34) (end 121.5 100.26) (width 0.5) (layer "F.Cu") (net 34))
 (segment (start 120.58 84.24) (end 120.58 99.34) (width 0.5) (layer "F.Cu") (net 34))
 (segment (start 76.5 133) (end 72 133) (width 0.5) (layer "F.Cu") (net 15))
 (segment (start 73.5 114.5) (end 79.5 114.5) (width 0.5) (layer "F.Cu") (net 15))
 (segment (start 73.5 124.96) (end 73.5 114.5) (width 0.5) (layer "F.Cu") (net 15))
 (segment (start 72 133) (end 71.5 132.5) (width 0.5) (layer "F.Cu") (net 15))
 (segment (start 95.18 132.5) (end 93.18 130.5) (width 0.5) (layer "F.Cu") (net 15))
 (segment (start 71.5 132.5) (end 71.5 126.96) (width 0.5) (layer "F.Cu") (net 15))
 (segment (start 79 130.5) (end 76.5 133) (width 0.5) (layer "F.Cu") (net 15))
 (segment (start 93.18 130.5) (end 79 130.5) (width 0.5) (layer "F.Cu") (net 15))
 (segment (start 71.5 126.96) (end 73.5 124.96) (width 0.5) (layer "F.Cu") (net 15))
 (segment (start 93.5 111) (end 93.5 88.5) (width 0.5) (layer "B.Cu") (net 15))
 (segment (start 93.5 88.5) (end 96.18 88.5) (width 0.5) (layer "B.Cu") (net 15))
 (segment (start 79.5 111) (end 93.5 111) (width 0.5) (layer "B.Cu") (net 15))
 (segment (start 79.5 114.5) (end 79.5 111) (width 0.5) (layer "B.Cu") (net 15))
 (segment (start 119 131.54) (end 119 118) (width 0.5) (layer "F.Cu") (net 40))
 (segment (start 118.04 132.5) (end 119 131.54) (width 0.5) (layer "F.Cu") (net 40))
 (segment (start 119 118) (end 121.5 115.5) (width 0.5) (layer "F.Cu") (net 40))
 (segment (start 97 82.5) (end 98.74 84.24) (width 0.5) (layer "F.Cu") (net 21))
 (segment (start 78.5 109.5) (end 68.5 109.5) (width 0.5) (layer "F.Cu") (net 21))
 (segment (start 82.5 105.5) (end 78.5 109.5) (width 0.5) (layer "F.Cu") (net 21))
 (segment (start 68.5 109.5) (end 68.5 82.5) (width 0.5) (layer "F.Cu") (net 21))
 (segment (start 68.5 82.5) (end 97 82.5) (width 0.5) (layer "F.Cu") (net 21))
 (segment (start 107.88 87.5) (end 108.88 88.5) (width 0.5) (layer "F.Cu") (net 11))
 (segment (start 107.88 84.24) (end 107.88 87.5) (width 0.5) (layer "F.Cu") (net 11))
 (segment (start 71 97.5) (end 71 92) (width 0.5) (layer "F.Cu") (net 20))
 (segment (start 71.5 98) (end 71 97.5) (width 0.5) (layer "F.Cu") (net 20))
 (segment (start 74 98) (end 71.5 98) (width 0.5) (layer "F.Cu") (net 20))
 (segment (start 73.54 93.54) (end 73.54 92) (width 0.5) (layer "F.Cu") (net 33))
 (segment (start 78 98) (end 73.54 93.54) (width 0.5) (layer "F.Cu") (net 33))
 (segment (start 82.5 95.88) (end 78.62 92) (width 0.5) (layer "F.Cu") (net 22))
 (segment (start 82.5 97.88) (end 82.5 95.88) (width 0.5) (layer "F.Cu") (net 22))
 (segment (start 114 104) (end 114 101) (width 0.5) (layer "F.Cu") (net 14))
 (segment (start 93.5 92) (end 93.5 104) (width 0.5) (layer "F.Cu") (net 14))
 (segment (start 98.72 88.5) (end 95.22 92) (width 0.5) (layer "F.Cu") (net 14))
 (segment (start 95.22 92) (end 93.5 92) (width 0.5) (layer "F.Cu") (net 14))
 (segment (start 93.5 104) (end 114 104) (width 0.5) (layer "F.Cu") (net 14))
 (segment (start 108.88 100.96) (end 108.92 101) (width 0.5) (layer "F.Cu") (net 6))
 (segment (start 108.88 96.12) (end 108.88 100.96) (width 0.5) (layer "F.Cu") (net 6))
 (segment (start 96.18 100.96) (end 96.22 101) (width 0.5) (layer "F.Cu") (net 1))
 (segment (start 96.18 96.12) (end 96.18 100.96) (width 0.5) (layer "F.Cu") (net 1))
 (segment (start 106.38 97.12) (end 106.38 101) (width 0.5) (layer "F.Cu") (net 5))
 (segment (start 106.34 96.12) (end 106.62 96.12) (width 0.5) (layer "F.Cu") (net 5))
 (segment (start 107 96.5) (end 106.38 97.12) (width 0.5) (layer "F.Cu") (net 5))
 (segment (start 106.62 96.12) (end 107 96.5) (width 0.5) (layer "F.Cu") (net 5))
 (segment (start 103.8 100.96) (end 103.84 101) (width 0.5) (layer "F.Cu") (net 4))
 (segment (start 103.8 96.12) (end 103.8 100.96) (width 0.5) (layer "F.Cu") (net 4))
 (segment (start 101.26 96.12) (end 101.26 100.96) (width 0.5) (layer "F.Cu") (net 3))
 (segment (start 101.26 100.96) (end 101.3 101) (width 0.5) (layer "F.Cu") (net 3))
 (segment (start 98.72 100.96) (end 98.76 101) (width 0.5) (layer "F.Cu") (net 2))
 (segment (start 98.72 96.12) (end 98.72 100.96) (width 0.5) (layer "F.Cu") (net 2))
 (segment (start 111.42 100.96) (end 111.46 101) (width 0.5) (layer "F.Cu") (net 7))
 (segment (start 111.42 96.12) (end 111.42 100.96) (width 0.5) (layer "F.Cu") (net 7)))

